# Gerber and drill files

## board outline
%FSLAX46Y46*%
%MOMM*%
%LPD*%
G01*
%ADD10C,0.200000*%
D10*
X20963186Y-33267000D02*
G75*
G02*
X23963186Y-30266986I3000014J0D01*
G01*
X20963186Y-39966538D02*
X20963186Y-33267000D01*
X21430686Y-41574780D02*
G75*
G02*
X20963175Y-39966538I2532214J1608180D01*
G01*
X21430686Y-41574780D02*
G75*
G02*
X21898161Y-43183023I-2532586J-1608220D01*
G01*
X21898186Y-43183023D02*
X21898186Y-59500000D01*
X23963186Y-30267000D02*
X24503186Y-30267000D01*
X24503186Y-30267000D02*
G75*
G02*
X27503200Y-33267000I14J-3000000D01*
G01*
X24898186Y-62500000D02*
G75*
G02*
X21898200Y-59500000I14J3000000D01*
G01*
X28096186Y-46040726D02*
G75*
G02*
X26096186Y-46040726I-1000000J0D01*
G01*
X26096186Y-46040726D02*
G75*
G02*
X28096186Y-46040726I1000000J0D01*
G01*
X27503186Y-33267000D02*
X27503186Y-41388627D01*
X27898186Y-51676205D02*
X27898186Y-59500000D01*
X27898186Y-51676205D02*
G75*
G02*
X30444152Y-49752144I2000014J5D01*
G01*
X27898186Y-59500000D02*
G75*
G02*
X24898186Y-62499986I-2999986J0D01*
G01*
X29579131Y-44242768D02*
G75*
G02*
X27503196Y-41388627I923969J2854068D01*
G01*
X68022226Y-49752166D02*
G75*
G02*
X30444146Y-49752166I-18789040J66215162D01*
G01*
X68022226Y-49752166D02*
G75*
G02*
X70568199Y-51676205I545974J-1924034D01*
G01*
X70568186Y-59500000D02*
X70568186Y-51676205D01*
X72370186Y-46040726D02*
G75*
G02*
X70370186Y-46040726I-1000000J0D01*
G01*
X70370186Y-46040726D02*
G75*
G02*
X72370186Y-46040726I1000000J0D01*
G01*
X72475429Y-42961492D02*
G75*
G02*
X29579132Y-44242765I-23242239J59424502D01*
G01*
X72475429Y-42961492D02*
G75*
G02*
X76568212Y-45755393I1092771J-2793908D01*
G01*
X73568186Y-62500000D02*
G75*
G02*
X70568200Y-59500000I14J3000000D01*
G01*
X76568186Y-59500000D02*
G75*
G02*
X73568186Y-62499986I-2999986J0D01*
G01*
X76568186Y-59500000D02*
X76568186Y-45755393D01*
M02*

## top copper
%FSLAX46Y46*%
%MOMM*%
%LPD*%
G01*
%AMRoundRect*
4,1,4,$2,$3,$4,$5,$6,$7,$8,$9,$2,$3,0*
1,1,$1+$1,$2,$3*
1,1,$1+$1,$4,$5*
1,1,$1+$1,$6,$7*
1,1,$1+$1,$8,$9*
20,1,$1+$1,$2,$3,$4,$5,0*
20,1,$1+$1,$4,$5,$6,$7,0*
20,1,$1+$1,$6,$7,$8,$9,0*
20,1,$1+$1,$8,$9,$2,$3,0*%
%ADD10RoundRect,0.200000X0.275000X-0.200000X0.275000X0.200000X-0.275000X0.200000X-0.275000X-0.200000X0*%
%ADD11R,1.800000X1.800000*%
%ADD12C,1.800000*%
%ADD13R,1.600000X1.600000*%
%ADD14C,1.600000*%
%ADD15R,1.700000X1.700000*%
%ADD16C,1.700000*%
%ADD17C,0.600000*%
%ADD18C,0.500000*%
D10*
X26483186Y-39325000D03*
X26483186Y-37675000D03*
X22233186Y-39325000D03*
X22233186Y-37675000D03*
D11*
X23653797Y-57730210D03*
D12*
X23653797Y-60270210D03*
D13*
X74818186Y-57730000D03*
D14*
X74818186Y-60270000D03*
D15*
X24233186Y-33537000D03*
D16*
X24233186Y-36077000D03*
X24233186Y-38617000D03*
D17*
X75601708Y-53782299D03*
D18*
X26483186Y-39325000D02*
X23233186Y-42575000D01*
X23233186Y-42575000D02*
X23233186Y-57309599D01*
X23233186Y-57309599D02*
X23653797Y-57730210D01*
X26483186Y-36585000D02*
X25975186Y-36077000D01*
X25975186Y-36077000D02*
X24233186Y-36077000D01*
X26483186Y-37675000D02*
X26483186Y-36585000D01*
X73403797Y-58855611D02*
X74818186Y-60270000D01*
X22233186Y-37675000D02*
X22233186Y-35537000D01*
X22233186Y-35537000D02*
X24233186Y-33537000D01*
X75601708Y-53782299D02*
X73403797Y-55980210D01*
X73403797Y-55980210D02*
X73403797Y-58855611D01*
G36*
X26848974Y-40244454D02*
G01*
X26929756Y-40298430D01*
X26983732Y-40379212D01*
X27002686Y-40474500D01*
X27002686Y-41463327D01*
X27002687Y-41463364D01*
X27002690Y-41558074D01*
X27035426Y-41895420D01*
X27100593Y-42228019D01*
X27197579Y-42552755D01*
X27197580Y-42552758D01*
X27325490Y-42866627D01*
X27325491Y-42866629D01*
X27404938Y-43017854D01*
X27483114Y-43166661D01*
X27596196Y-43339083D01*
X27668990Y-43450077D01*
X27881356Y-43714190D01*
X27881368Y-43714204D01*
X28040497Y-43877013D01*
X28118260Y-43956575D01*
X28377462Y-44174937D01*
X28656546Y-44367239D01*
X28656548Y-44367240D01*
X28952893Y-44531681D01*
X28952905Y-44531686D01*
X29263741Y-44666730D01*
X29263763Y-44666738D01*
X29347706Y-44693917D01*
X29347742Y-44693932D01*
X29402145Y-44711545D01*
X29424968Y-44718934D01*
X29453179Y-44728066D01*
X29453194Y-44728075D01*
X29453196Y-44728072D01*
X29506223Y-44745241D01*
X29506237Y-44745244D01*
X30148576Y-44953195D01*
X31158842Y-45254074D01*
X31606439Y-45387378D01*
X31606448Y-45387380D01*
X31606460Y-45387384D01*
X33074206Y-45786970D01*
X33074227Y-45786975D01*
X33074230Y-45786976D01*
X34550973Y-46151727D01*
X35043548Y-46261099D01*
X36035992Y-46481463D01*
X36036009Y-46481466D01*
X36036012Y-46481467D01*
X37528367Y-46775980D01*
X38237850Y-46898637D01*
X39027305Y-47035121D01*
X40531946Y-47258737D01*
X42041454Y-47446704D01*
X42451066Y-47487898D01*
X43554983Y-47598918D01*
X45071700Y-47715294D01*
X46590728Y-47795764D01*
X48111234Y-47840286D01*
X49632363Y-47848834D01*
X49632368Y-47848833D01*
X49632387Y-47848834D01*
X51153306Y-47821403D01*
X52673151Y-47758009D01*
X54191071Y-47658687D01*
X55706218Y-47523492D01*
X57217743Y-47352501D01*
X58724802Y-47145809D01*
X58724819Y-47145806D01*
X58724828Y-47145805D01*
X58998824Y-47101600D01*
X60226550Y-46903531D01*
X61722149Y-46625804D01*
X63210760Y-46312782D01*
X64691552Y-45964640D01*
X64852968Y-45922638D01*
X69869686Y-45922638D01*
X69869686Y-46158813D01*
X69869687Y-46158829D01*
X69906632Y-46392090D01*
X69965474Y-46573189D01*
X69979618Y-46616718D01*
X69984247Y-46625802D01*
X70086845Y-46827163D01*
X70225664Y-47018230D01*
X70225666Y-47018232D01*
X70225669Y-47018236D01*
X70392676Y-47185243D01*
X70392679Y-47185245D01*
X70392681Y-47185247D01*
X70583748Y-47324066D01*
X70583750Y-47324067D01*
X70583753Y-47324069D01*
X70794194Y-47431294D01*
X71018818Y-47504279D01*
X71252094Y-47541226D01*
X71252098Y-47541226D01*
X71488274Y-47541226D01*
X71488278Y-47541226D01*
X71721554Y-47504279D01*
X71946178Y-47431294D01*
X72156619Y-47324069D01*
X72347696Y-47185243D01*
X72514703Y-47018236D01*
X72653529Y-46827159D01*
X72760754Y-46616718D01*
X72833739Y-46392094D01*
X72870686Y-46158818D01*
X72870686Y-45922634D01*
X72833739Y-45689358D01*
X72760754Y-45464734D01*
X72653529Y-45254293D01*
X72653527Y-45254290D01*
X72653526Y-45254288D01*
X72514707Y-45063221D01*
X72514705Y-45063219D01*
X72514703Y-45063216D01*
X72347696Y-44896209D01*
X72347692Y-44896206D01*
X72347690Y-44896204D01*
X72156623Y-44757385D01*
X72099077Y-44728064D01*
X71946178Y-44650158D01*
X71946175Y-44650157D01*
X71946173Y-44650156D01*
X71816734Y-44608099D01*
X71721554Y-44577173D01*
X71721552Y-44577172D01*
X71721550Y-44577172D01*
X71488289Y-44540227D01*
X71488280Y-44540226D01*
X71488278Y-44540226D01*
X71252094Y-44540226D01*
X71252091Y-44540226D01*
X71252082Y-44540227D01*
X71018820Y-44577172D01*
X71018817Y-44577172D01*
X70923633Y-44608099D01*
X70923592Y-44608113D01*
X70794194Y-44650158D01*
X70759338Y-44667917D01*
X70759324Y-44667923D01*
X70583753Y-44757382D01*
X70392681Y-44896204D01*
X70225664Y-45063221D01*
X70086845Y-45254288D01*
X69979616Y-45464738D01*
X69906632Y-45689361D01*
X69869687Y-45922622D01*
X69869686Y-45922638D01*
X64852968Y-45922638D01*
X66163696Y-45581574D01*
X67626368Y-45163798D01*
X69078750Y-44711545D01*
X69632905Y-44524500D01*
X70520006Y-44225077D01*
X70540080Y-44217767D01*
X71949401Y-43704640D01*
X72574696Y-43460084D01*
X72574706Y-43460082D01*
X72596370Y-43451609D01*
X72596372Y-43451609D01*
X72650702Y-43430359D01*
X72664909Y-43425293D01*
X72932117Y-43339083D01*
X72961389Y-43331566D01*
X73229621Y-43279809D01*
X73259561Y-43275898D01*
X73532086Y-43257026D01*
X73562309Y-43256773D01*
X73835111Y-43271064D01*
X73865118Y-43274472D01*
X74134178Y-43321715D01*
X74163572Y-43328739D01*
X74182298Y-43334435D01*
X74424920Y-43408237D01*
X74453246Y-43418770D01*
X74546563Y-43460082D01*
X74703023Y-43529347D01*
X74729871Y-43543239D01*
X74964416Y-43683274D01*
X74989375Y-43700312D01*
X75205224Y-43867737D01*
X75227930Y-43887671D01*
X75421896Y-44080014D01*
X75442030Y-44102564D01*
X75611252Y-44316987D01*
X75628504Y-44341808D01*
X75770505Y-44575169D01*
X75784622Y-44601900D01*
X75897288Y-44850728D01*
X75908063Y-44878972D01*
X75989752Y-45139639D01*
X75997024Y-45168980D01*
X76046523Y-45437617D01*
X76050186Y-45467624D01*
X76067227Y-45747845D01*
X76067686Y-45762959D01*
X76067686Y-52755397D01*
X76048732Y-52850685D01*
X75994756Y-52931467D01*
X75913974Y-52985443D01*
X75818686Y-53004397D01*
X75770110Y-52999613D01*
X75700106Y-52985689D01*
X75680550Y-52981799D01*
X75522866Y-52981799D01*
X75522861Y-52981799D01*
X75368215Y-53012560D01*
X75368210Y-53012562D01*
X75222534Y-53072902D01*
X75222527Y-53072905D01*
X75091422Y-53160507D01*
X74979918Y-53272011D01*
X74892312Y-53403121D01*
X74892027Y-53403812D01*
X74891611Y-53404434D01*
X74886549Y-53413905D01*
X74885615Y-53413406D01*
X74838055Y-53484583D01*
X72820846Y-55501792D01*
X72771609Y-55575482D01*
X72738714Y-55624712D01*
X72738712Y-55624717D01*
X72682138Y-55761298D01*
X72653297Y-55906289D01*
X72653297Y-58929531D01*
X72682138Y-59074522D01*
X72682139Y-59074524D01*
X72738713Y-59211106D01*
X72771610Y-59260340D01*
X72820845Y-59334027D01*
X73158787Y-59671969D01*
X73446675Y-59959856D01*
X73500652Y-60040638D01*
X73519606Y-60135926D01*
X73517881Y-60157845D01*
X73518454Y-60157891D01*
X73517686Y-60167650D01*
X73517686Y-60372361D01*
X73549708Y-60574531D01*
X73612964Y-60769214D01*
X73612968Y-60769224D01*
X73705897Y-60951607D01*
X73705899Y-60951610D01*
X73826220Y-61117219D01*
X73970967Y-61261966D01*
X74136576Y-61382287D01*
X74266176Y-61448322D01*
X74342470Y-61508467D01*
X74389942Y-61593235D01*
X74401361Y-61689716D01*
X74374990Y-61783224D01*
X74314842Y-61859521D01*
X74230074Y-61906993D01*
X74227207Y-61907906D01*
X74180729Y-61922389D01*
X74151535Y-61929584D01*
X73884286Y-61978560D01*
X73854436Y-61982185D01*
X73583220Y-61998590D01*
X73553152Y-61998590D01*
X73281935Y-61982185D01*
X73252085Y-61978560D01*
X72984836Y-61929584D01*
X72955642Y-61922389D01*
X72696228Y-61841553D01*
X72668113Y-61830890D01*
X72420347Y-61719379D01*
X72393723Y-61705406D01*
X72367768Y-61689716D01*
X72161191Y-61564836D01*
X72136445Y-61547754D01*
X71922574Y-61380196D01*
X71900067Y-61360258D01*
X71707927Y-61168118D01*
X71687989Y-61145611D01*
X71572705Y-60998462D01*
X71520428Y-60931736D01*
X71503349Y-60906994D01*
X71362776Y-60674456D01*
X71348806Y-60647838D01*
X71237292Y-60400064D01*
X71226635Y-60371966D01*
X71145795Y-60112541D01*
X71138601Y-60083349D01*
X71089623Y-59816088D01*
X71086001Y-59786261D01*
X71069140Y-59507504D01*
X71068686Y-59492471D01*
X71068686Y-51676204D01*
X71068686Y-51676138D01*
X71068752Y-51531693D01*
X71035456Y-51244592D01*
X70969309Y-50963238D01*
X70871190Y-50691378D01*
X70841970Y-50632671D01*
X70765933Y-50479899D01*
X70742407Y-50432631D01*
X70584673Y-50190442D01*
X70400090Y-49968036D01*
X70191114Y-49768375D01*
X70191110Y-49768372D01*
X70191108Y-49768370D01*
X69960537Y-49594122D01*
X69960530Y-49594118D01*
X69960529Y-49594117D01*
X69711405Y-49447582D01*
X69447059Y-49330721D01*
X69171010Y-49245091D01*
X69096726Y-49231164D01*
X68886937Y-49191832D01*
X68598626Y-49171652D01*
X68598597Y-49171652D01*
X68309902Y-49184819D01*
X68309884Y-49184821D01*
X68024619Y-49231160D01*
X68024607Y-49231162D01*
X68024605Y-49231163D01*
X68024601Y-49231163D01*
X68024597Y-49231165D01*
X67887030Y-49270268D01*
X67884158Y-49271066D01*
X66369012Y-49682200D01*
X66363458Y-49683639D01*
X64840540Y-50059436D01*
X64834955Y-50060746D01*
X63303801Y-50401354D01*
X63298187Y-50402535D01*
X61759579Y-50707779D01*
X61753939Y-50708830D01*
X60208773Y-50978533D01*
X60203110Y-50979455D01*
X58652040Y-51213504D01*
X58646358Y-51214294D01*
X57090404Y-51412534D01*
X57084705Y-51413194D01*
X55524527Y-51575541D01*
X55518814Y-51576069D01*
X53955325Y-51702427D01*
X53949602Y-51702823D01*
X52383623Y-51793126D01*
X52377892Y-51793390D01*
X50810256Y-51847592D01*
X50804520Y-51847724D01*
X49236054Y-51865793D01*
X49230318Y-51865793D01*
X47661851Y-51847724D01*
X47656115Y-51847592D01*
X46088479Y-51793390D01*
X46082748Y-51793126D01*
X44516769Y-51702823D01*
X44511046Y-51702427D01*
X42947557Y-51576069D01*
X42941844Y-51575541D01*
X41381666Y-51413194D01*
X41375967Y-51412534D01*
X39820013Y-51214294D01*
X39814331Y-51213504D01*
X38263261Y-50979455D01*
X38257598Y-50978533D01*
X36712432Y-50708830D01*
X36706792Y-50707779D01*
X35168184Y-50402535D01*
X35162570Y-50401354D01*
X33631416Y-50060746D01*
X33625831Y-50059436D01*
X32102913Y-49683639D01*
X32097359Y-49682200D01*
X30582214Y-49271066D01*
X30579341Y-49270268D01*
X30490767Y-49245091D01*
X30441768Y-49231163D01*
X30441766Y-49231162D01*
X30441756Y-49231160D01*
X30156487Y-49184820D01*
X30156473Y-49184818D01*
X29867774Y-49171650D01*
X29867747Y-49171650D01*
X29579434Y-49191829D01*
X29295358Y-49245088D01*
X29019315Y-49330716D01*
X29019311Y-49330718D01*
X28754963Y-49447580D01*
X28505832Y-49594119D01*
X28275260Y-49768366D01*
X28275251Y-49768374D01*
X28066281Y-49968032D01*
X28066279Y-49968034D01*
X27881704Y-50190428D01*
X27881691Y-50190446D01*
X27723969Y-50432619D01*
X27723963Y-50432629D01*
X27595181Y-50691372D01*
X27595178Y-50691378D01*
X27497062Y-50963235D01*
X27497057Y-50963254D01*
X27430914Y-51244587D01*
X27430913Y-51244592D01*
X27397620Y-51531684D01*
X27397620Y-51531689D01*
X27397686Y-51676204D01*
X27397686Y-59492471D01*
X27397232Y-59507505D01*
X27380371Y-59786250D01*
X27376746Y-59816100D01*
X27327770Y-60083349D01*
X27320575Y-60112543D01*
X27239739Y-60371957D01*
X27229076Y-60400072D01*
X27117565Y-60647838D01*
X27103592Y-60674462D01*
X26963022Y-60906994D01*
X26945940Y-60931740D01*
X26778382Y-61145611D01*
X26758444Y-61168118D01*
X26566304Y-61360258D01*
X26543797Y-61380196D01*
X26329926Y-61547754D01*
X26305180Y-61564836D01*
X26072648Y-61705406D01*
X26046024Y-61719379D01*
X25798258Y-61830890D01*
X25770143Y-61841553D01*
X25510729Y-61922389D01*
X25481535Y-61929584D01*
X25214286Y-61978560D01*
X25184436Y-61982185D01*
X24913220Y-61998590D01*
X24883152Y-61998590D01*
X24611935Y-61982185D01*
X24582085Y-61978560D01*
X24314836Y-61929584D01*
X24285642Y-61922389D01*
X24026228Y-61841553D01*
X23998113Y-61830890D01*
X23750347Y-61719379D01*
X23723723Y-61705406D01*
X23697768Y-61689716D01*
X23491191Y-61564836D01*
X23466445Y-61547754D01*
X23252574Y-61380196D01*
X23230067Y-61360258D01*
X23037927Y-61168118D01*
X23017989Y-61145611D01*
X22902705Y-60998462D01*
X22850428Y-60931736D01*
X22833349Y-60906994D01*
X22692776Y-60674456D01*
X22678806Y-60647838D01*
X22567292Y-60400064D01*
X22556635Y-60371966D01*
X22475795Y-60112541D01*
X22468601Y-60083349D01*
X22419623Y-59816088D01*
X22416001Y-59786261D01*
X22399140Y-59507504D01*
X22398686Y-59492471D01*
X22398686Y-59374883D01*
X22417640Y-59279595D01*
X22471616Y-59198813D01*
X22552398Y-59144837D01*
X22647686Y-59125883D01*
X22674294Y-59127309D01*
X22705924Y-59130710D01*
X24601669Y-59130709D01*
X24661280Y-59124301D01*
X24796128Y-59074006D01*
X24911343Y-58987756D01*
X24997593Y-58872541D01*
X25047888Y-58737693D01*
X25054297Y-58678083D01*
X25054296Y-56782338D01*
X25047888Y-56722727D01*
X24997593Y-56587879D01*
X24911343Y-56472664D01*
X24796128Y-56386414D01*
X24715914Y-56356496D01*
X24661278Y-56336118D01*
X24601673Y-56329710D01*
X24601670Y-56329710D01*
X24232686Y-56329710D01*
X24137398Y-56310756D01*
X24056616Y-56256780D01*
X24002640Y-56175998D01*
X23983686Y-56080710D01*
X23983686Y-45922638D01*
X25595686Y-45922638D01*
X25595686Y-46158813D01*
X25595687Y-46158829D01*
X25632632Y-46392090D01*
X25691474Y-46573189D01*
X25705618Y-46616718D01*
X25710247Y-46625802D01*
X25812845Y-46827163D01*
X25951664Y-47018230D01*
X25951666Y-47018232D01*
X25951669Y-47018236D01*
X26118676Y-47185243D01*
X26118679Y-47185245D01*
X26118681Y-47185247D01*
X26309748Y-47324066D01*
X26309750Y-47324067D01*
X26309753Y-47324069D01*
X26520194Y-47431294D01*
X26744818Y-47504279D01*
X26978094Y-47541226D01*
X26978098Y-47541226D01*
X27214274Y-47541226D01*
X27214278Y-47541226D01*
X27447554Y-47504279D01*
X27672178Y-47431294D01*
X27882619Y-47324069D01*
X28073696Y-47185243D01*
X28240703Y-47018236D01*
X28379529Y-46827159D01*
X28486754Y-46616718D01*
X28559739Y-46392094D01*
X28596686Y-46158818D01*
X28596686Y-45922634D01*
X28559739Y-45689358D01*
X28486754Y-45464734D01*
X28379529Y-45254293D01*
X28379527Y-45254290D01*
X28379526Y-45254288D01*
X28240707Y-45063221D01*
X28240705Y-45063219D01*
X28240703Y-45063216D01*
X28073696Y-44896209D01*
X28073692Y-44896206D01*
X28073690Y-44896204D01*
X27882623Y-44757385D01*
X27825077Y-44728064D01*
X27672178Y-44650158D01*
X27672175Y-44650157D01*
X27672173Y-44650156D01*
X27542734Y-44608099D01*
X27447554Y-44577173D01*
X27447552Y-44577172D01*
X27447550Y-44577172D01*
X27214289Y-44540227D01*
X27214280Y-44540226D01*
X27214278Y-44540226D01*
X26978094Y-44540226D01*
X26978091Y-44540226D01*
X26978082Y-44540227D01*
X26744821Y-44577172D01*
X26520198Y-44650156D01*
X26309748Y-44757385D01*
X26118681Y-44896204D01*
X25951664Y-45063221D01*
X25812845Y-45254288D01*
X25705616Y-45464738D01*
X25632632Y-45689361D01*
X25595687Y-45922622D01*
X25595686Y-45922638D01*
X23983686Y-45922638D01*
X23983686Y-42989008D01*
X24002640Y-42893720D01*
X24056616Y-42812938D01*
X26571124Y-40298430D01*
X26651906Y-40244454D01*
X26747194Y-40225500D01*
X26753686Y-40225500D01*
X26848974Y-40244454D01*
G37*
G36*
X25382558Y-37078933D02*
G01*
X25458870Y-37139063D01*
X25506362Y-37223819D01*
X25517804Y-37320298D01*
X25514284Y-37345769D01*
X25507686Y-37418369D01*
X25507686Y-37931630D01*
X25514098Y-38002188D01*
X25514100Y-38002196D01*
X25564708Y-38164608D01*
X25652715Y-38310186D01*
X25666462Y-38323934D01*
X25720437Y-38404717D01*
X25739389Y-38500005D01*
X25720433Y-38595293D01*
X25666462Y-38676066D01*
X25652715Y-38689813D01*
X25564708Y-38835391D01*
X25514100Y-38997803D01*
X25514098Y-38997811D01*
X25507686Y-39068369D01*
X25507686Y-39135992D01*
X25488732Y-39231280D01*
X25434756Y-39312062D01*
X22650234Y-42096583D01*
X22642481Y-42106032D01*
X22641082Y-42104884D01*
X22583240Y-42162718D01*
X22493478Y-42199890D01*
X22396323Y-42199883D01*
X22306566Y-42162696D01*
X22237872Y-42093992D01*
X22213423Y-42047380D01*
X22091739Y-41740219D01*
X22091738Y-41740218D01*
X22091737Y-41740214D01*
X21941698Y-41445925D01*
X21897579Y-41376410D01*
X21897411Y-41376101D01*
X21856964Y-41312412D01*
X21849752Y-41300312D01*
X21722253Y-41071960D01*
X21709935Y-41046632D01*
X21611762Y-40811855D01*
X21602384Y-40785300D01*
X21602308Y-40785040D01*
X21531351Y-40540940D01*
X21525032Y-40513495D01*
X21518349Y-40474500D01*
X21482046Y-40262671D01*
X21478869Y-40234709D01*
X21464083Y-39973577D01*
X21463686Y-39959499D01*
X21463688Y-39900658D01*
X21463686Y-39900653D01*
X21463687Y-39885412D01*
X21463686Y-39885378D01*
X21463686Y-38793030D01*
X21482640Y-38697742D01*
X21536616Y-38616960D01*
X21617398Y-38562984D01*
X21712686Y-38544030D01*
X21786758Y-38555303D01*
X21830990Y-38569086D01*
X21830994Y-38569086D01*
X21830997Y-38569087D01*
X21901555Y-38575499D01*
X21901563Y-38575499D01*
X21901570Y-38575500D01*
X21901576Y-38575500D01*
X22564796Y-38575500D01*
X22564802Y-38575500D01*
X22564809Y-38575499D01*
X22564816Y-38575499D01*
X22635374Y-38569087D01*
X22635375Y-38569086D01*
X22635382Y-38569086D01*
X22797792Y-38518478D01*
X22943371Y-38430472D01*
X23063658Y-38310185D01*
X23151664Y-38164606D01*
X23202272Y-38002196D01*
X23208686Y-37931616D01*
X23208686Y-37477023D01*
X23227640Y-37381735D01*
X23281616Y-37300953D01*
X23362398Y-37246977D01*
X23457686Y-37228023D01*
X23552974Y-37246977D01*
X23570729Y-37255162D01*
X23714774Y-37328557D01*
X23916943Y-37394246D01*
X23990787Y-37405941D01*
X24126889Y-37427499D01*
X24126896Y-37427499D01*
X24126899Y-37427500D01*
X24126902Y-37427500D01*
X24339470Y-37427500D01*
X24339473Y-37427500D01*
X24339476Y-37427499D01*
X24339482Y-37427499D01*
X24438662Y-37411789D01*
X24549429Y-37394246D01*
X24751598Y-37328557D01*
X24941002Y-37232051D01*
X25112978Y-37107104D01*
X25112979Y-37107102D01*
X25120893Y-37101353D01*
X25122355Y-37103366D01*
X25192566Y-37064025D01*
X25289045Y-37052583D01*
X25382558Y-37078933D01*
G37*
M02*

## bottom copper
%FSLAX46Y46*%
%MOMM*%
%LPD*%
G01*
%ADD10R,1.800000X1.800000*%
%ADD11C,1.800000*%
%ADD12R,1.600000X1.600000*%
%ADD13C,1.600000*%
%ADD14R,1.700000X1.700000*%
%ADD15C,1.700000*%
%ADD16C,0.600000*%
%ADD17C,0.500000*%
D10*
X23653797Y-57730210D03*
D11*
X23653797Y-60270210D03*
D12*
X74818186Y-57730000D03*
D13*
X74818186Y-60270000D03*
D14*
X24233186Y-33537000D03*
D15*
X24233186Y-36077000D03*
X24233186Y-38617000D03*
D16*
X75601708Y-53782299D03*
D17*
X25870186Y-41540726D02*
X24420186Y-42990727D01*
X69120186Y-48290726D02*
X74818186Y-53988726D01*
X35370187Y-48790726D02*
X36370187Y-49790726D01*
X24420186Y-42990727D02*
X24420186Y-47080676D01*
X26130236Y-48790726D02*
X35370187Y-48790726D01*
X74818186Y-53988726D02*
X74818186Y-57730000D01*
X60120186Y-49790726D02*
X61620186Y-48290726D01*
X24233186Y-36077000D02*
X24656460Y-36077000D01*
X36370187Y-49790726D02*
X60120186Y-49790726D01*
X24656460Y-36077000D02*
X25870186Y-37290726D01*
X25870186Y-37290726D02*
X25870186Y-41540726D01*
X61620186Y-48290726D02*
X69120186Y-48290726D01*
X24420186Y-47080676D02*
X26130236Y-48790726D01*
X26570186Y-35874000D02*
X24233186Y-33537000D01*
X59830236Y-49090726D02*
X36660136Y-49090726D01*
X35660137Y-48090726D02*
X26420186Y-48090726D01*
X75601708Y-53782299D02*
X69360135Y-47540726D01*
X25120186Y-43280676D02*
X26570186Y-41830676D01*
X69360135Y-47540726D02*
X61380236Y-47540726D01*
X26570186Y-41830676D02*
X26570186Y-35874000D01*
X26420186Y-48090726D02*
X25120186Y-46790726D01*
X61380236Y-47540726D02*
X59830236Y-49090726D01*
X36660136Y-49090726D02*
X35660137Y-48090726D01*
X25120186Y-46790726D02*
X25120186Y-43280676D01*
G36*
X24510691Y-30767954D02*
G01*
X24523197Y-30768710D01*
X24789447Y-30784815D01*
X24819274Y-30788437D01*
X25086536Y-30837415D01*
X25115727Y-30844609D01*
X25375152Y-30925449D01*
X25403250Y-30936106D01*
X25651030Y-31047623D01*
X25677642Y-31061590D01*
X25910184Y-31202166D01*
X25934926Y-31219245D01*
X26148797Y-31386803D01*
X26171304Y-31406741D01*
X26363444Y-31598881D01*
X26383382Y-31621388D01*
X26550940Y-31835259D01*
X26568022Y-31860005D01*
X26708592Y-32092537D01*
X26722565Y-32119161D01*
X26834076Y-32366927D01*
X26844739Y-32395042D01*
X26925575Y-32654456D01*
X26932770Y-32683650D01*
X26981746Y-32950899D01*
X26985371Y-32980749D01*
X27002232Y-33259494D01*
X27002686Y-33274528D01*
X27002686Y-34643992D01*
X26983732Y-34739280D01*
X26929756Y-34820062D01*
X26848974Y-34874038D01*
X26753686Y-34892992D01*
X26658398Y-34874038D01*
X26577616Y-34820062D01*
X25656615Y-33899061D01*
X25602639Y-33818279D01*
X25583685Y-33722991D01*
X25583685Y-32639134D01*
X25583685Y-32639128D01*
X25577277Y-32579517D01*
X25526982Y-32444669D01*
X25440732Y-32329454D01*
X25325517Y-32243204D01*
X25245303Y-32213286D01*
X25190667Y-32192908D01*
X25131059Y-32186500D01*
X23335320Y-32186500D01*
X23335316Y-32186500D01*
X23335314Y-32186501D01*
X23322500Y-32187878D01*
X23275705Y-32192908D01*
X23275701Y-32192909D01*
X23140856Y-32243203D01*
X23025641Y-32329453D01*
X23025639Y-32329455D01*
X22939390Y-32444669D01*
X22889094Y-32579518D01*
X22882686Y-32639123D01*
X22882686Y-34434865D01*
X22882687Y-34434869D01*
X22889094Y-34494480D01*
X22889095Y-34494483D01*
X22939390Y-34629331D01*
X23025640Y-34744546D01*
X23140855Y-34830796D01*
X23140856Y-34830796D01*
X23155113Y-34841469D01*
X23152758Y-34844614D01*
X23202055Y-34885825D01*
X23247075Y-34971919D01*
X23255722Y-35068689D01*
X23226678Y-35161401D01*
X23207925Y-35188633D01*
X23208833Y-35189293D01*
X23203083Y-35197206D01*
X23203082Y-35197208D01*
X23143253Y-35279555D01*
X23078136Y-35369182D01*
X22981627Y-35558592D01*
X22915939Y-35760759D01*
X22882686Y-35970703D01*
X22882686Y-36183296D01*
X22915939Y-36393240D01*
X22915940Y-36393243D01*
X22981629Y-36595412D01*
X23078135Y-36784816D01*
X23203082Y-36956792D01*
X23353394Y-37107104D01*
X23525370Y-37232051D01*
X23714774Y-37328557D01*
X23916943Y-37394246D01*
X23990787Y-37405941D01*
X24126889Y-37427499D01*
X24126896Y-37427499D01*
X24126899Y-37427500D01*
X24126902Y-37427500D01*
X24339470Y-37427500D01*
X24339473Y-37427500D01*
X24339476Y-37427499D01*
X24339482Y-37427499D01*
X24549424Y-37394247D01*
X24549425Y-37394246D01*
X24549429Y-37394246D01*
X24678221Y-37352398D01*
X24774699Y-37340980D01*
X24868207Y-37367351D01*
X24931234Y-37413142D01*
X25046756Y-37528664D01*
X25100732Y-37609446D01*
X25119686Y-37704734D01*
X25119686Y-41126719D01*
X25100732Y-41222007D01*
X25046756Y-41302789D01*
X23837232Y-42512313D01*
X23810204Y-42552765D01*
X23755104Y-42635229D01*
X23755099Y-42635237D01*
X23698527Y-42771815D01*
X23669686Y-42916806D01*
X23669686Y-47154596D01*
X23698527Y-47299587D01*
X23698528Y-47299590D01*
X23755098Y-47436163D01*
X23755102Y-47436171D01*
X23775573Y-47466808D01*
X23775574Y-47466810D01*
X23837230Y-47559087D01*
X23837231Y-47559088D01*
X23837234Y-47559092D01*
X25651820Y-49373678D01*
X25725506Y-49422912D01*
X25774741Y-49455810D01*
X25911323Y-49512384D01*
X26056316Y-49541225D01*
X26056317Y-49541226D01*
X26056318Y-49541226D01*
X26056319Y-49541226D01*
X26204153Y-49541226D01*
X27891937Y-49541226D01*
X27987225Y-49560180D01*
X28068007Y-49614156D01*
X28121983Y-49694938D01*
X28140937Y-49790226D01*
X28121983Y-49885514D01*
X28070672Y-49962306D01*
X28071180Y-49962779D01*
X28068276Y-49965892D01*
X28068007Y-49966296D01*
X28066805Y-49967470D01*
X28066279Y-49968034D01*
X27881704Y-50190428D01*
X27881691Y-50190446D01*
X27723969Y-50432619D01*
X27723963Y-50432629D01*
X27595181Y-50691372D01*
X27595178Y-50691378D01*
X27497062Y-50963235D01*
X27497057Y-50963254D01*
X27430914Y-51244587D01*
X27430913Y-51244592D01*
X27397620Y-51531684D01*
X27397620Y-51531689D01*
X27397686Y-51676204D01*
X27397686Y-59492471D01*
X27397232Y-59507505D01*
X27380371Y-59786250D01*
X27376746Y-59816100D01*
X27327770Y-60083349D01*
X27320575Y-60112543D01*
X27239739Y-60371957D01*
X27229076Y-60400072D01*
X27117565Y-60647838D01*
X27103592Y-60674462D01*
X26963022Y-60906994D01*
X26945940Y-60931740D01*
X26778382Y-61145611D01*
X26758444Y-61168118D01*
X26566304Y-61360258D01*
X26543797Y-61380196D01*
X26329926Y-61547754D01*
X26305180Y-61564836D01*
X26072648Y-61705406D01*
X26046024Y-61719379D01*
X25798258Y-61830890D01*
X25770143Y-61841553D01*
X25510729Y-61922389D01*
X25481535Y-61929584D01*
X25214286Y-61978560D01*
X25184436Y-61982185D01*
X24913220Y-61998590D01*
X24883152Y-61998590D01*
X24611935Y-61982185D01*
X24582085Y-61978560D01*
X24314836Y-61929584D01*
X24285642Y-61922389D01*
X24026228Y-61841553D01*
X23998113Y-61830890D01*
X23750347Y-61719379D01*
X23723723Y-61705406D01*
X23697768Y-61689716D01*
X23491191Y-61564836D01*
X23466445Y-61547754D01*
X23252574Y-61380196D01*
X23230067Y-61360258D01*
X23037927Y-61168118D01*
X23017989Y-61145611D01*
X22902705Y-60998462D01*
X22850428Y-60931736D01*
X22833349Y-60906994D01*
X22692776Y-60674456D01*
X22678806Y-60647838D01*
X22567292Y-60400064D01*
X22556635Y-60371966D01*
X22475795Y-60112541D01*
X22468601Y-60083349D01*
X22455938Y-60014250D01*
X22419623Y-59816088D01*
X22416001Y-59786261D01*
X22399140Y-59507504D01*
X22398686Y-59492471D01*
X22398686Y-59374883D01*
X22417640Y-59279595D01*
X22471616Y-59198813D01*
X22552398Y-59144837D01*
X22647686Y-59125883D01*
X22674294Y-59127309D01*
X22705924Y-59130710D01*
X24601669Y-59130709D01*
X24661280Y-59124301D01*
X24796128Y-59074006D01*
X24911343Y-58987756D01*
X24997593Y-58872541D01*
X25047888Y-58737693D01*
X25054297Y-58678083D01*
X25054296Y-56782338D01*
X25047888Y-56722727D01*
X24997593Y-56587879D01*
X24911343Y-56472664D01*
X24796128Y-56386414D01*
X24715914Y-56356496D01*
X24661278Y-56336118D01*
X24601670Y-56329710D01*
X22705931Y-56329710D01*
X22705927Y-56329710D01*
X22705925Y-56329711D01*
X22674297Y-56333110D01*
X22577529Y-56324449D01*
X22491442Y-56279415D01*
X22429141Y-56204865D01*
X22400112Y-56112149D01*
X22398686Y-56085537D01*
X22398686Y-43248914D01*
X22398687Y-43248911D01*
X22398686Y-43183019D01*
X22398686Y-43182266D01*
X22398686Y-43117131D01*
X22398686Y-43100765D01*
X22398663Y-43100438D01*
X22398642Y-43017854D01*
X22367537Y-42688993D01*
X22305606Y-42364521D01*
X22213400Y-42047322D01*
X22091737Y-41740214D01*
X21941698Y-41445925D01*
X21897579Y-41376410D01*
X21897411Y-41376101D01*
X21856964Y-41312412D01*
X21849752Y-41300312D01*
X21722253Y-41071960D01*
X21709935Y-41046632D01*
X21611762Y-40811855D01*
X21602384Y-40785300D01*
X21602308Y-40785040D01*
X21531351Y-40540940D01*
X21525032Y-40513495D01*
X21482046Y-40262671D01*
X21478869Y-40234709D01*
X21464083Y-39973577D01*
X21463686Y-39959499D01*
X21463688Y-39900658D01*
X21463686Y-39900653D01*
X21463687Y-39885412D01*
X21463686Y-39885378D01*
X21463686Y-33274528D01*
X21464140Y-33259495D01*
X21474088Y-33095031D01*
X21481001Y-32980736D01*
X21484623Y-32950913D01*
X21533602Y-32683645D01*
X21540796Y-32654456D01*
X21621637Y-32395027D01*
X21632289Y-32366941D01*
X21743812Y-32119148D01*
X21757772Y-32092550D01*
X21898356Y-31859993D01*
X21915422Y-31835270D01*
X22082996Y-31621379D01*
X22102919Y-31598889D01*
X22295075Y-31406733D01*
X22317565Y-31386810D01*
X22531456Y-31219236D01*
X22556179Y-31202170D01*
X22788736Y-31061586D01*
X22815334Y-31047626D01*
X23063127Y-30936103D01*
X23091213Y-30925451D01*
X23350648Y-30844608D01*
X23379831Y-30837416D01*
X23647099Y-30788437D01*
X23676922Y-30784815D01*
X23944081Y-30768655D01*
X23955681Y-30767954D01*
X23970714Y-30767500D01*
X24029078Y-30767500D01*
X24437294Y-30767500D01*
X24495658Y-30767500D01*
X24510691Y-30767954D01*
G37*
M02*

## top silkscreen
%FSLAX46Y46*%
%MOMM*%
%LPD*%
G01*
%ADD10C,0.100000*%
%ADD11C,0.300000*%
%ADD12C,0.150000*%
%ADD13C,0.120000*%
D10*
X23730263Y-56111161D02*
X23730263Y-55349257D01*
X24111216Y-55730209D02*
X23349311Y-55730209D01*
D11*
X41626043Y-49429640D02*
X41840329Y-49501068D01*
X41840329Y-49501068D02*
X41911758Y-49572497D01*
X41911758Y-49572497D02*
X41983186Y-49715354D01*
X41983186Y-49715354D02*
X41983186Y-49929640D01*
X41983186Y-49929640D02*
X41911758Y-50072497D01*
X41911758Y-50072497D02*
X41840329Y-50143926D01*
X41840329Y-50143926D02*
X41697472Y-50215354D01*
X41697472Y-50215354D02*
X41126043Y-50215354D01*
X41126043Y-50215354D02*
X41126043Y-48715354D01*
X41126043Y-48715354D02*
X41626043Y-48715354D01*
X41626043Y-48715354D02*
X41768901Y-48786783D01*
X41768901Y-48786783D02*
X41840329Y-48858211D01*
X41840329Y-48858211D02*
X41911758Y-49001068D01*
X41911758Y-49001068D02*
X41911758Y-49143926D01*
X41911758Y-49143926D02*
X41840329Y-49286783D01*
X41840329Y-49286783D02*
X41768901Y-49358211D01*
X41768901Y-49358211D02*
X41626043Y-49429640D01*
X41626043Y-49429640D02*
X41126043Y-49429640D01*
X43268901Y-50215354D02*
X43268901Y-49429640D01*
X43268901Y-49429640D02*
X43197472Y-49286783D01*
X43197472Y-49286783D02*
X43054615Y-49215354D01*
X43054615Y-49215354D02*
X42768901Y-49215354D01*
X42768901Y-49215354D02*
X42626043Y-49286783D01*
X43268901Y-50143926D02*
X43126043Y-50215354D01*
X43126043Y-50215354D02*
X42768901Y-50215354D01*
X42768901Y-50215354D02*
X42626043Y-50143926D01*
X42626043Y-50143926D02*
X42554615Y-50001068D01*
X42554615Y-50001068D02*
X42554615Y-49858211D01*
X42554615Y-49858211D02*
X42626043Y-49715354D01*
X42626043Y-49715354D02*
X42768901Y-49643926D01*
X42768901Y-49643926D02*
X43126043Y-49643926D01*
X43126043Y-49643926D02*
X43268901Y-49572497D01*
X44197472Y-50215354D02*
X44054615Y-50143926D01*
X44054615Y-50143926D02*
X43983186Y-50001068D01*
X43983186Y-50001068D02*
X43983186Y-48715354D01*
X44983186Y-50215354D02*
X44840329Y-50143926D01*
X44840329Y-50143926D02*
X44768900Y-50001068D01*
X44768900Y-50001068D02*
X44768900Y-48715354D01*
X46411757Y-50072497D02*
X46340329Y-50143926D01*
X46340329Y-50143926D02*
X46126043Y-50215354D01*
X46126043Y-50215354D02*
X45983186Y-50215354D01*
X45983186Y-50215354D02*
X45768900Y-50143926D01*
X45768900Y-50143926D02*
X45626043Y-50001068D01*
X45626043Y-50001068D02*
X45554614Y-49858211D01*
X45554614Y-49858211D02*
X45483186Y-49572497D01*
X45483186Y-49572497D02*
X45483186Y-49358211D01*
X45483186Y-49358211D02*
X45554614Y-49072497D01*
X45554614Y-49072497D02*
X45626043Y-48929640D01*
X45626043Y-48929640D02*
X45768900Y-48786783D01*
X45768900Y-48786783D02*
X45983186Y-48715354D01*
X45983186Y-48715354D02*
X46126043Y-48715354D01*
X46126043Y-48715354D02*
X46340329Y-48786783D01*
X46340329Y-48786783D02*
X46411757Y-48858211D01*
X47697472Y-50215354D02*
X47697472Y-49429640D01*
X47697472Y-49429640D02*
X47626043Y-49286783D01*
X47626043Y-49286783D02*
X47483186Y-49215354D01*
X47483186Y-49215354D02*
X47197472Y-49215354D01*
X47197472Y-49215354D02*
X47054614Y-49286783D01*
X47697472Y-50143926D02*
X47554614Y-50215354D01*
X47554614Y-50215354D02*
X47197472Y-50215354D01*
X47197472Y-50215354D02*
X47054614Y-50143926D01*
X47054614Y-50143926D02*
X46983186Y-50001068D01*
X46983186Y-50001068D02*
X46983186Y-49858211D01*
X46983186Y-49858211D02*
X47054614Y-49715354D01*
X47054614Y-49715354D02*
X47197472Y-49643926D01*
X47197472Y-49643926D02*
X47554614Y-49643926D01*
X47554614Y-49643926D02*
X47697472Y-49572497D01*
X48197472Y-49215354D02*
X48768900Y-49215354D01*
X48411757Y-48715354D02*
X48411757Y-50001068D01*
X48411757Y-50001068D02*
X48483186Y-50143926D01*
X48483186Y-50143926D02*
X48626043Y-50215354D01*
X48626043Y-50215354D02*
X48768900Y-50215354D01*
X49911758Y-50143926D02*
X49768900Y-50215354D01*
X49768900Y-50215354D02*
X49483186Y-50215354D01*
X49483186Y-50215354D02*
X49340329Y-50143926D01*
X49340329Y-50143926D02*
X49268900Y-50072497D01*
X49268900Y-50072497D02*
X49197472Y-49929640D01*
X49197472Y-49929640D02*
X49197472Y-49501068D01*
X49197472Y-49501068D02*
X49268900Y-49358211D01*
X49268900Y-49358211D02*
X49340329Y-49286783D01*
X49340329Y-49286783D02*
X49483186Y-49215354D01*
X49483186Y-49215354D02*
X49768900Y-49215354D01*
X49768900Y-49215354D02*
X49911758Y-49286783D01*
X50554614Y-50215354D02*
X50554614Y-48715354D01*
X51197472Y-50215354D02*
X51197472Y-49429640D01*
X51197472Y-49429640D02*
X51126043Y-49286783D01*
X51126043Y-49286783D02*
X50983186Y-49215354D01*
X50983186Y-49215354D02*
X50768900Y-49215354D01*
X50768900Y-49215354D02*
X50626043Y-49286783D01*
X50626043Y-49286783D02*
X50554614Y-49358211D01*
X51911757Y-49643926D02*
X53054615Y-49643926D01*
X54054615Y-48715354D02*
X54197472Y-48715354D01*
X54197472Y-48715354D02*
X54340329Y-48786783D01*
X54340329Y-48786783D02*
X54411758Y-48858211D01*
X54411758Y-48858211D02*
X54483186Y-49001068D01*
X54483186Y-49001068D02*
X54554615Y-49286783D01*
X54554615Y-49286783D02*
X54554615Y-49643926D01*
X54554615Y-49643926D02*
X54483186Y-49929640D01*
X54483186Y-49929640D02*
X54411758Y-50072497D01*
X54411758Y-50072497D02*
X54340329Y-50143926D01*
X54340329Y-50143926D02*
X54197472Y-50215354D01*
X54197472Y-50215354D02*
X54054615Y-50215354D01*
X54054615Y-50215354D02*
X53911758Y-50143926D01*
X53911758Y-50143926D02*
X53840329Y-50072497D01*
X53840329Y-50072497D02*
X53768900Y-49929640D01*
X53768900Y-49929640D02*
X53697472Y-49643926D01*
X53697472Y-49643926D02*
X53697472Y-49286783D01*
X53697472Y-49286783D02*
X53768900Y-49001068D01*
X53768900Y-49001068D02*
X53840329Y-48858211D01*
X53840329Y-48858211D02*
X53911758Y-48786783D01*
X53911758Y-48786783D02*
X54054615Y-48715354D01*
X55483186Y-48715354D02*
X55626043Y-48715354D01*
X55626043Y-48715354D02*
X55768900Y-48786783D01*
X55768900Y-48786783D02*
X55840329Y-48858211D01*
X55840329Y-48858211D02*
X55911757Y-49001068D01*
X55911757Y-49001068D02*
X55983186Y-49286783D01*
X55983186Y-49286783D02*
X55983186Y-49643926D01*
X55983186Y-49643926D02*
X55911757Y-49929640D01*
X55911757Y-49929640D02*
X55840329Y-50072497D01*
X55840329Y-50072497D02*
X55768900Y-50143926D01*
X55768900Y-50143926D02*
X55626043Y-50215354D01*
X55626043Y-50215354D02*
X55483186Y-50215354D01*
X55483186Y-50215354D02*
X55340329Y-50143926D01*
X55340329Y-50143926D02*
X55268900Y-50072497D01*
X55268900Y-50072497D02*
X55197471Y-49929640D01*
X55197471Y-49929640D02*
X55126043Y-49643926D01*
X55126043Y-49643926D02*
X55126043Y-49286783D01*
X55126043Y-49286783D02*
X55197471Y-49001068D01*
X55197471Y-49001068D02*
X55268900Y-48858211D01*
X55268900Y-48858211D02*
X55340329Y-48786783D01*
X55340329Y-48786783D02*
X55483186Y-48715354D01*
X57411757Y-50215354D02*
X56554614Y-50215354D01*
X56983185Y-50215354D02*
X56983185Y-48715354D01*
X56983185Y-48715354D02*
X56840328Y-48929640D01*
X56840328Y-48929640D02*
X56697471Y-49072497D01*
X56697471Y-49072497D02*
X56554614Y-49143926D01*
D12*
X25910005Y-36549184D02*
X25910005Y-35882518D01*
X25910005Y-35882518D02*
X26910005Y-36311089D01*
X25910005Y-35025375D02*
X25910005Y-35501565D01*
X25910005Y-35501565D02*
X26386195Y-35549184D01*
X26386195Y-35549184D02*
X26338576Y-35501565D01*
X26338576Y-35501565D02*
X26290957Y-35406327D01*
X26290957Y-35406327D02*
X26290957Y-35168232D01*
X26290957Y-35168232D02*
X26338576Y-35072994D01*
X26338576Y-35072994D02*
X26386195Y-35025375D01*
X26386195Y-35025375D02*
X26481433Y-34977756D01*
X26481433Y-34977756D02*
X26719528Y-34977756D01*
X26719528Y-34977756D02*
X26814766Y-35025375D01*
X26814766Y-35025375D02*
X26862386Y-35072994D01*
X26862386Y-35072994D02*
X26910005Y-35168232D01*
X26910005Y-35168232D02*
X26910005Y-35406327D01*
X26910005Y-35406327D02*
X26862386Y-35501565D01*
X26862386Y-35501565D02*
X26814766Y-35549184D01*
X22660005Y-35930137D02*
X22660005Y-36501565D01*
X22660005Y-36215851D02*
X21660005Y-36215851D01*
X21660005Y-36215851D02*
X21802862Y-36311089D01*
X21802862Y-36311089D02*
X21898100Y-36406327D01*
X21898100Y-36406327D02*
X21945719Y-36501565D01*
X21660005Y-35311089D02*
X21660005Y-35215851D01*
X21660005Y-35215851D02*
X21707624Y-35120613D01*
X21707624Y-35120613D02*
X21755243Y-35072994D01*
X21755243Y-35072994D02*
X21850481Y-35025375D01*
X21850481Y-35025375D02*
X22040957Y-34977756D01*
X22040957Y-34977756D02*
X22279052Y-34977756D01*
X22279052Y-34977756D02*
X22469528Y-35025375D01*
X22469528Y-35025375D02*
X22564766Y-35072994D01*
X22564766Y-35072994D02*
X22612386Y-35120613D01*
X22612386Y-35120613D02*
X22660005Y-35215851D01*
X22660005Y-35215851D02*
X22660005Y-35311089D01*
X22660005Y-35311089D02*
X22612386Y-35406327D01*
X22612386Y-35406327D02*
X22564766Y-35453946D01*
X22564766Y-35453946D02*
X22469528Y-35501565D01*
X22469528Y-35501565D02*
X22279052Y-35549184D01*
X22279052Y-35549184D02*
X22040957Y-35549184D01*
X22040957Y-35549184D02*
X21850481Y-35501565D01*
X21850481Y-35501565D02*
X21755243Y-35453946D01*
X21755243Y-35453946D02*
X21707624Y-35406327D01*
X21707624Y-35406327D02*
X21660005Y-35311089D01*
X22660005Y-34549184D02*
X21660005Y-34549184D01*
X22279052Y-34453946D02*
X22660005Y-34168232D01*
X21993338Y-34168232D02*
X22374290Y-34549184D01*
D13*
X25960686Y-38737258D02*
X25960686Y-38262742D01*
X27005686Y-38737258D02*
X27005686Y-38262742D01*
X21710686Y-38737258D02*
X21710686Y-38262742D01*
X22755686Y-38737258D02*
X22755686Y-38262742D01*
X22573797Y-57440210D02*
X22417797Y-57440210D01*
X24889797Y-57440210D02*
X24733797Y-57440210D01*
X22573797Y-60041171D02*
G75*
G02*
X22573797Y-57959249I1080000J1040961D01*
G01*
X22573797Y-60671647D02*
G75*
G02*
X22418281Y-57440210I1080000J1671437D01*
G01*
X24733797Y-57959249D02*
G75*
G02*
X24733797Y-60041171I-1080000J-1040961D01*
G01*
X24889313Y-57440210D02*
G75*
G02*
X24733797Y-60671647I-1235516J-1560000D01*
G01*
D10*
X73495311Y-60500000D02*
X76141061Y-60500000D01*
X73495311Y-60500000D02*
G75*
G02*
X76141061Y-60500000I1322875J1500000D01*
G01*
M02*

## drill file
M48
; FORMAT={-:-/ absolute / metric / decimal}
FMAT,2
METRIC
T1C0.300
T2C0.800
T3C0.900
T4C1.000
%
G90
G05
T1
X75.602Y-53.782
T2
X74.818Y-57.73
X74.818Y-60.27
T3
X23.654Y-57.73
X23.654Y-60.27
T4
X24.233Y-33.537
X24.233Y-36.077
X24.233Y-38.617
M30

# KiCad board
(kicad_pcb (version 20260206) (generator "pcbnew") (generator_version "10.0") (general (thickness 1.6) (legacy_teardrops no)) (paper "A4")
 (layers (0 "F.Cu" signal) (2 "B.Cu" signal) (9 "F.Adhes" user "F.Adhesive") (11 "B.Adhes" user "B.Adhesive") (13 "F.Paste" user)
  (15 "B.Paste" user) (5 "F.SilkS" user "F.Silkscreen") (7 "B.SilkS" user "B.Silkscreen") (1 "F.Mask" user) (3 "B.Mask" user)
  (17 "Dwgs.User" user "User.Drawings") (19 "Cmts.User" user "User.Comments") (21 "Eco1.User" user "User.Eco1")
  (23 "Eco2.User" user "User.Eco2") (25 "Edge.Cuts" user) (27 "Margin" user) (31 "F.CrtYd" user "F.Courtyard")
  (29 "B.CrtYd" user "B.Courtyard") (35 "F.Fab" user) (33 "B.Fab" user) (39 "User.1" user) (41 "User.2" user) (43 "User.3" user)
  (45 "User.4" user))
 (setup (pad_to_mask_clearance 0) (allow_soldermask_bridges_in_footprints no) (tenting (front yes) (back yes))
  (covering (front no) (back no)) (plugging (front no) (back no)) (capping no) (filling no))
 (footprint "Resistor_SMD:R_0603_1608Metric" (layer "F.Cu") (at 26.483186 38.5 90)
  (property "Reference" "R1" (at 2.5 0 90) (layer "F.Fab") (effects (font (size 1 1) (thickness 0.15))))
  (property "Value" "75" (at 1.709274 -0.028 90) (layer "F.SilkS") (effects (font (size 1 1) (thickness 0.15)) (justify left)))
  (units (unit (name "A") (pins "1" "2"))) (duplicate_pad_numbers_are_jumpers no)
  (fp_line (start -0.237258 -0.5225) (end 0.237258 -0.5225) (stroke (width 0.12) (type solid)) (layer "F.SilkS"))
  (fp_line (start -0.237258 0.5225) (end 0.237258 0.5225) (stroke (width 0.12) (type solid)) (layer "F.SilkS"))
  (pad "1" smd roundrect (at -0.825 0 90) (size 0.8 0.95) (layers "F.Cu" "F.Mask" "F.Paste") (roundrect_rratio 0.25) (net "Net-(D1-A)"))
  (pad "2" smd roundrect (at 0.825 0 90) (size 0.8 0.95) (layers "F.Cu" "F.Mask" "F.Paste") (roundrect_rratio 0.25) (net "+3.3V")))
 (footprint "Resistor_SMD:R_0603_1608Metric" (layer "F.Cu") (at 22.233186 38.5 90)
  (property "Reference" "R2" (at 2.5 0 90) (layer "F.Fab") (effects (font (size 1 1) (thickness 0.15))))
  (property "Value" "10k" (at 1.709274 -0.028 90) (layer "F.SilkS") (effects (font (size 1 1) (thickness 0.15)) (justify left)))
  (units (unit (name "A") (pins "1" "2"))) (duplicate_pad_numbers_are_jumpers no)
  (fp_line (start -0.237258 -0.5225) (end 0.237258 -0.5225) (stroke (width 0.12) (type solid)) (layer "F.SilkS"))
  (fp_line (start -0.237258 0.5225) (end 0.237258 0.5225) (stroke (width 0.12) (type solid)) (layer "F.SilkS"))
  (pad "1" smd roundrect (at -0.825 0 90) (size 0.8 0.95) (layers "F.Cu" "F.Mask" "F.Paste") (roundrect_rratio 0.25) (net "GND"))
  (pad "2" smd roundrect (at 0.825 0 90) (size 0.8 0.95) (layers "F.Cu" "F.Mask" "F.Paste") (roundrect_rratio 0.25) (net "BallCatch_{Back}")))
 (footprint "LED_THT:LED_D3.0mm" (layer "F.Cu") (at 23.653797 57.73021 -90)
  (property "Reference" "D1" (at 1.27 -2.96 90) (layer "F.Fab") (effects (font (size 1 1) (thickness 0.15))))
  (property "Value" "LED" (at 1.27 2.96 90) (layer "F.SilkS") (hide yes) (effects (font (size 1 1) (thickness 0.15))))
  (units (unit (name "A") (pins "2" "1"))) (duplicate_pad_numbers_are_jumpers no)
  (fp_line (start -0.29 1.08) (end -0.29 1.236) (stroke (width 0.12) (type solid)) (layer "F.SilkS"))
  (fp_line (start -0.29 -1.236) (end -0.29 -1.08) (stroke (width 0.12) (type solid)) (layer "F.SilkS"))
  (fp_arc (start 2.310961 1.08) (mid 1.27 1.5) (end 0.229039 1.08) (stroke (width 0.12) (type solid)) (layer "F.SilkS"))
  (fp_arc (start 2.941437 1.08) (mid 1.36566 1.987699) (end -0.29 1.235516) (stroke (width 0.12) (type solid)) (layer "F.SilkS"))
  (fp_arc (start 0.229039 -1.08) (mid 1.27 -1.5) (end 2.310961 -1.08) (stroke (width 0.12) (type solid)) (layer "F.SilkS"))
  (fp_arc (start -0.29 -1.235516) (mid 1.36566 -1.987699) (end 2.941437 -1.08) (stroke (width 0.12) (type solid)) (layer "F.SilkS"))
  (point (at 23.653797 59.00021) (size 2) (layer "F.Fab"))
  (pad "1" thru_hole rect (at 0 0 270) (size 1.8 1.8) (drill 0.9) (layers "*.Cu" "*.Mask") (remove_unused_layers no) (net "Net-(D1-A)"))
  (pad "2" thru_hole circle (at 2.54 0 270) (size 1.8 1.8) (drill 0.9) (layers "*.Cu" "*.Mask") (remove_unused_layers no) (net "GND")))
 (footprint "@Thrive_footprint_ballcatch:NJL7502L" (layer "F.Cu") (at 74.818186 59 90)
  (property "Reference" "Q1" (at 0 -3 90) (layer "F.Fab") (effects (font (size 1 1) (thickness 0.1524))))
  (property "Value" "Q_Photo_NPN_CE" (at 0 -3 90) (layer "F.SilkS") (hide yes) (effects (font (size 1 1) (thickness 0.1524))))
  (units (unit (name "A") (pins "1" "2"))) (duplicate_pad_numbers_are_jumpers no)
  (fp_line (start -1.5 -1.322875) (end -1.5 1.322875) (stroke (width 0.1) (type default)) (layer "F.SilkS"))
  (fp_arc (start -1.5 -1.322875) (mid 2 0) (end -1.5 1.322875) (stroke (width 0.1) (type default)) (layer "F.SilkS"))
  (pad "1" thru_hole rect (at 1.27 0 180) (size 1.6 1.6) (drill 0.8) (layers "*.Cu" "*.Mask") (remove_unused_layers no) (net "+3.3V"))
  (pad "2" thru_hole circle (at -1.27 0 180) (size 1.6 1.6) (drill 0.8) (layers "*.Cu" "*.Mask") (remove_unused_layers no)
   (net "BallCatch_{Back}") (thermal_bridge_angle 90)))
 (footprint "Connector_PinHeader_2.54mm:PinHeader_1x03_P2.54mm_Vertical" (layer "B.Cu") (at 24.233186 33.537 180)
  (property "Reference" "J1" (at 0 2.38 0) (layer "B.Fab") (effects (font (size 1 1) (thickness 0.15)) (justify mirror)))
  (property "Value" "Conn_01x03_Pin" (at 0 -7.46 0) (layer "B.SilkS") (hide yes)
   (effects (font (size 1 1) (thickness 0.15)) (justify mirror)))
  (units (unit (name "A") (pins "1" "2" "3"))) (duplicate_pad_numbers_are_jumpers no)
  (pad "1" thru_hole rect (at 0 0 180) (size 1.7 1.7) (drill 1) (layers "*.Cu" "*.Mask") (remove_unused_layers no) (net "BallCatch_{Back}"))
  (pad "2" thru_hole circle (at 0 -2.54 180) (size 1.7 1.7) (drill 1) (layers "*.Cu" "*.Mask") (remove_unused_layers no) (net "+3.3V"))
  (pad "3" thru_hole circle (at 0 -5.08 180) (size 1.7 1.7) (drill 1) (layers "*.Cu" "*.Mask") (remove_unused_layers no) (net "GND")))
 (gr_arc (start 20.963186 33.267) (mid 21.841866 31.14568) (end 23.963186 30.267) (stroke (width 0.2) (type default)) (layer "Edge.Cuts"))
 (gr_line (start 20.963186 39.966538) (end 20.963186 33.267) (stroke (width 0.2) (type default)) (layer "Edge.Cuts"))
 (gr_arc (start 21.430686 41.57478) (mid 21.082421 40.803946) (end 20.963186 39.966538) (stroke (width 0.2) (type default))
  (layer "Edge.Cuts"))
 (gr_arc (start 21.430686 41.57478) (mid 21.778938 42.345618) (end 21.898186 43.183023) (stroke (width 0.2) (type default))
  (layer "Edge.Cuts"))
 (gr_line (start 21.898186 43.183023) (end 21.898186 59.5) (stroke (width 0.2) (type default)) (layer "Edge.Cuts"))
 (gr_line (start 23.963186 30.267) (end 24.503186 30.267) (stroke (width 0.2) (type default)) (layer "Edge.Cuts"))
 (gr_arc (start 24.503186 30.267) (mid 26.624506 31.14568) (end 27.503186 33.267) (stroke (width 0.2) (type default)) (layer "Edge.Cuts"))
 (gr_arc (start 24.898186 62.5) (mid 22.776866 61.62132) (end 21.898186 59.5) (stroke (width 0.2) (type default)) (layer "Edge.Cuts"))
 (gr_circle (center 27.096186 46.040726) (end 26.096186 46.040726) (stroke (width 0.2) (type default)) (fill no) (layer "Edge.Cuts"))
 (gr_line (start 27.503186 33.267) (end 27.503186 41.388627) (stroke (width 0.2) (type default)) (layer "Edge.Cuts"))
 (gr_line (start 27.898186 51.676205) (end 27.898186 59.5) (stroke (width 0.2) (type default)) (layer "Edge.Cuts"))
 (gr_arc (start 27.898186 51.676205) (mid 28.692349 50.080595) (end 30.444146 49.752166) (stroke (width 0.2) (type default))
  (layer "Edge.Cuts"))
 (gr_arc (start 27.898186 59.5) (mid 27.019506 61.62132) (end 24.898186 62.5) (stroke (width 0.2) (type default)) (layer "Edge.Cuts"))
 (gr_arc (start 29.579131 44.242768) (mid 28.077051 43.153259) (end 27.503186 41.388627) (stroke (width 0.2) (type default))
  (layer "Edge.Cuts"))
 (gr_arc (start 68.022226 49.752166) (mid 49.233186 52.366327) (end 30.444146 49.752166) (stroke (width 0.2) (type default))
  (layer "Edge.Cuts"))
 (gr_arc (start 68.022226 49.752166) (mid 69.774022 50.080599) (end 70.568186 51.676205) (stroke (width 0.2) (type default))
  (layer "Edge.Cuts"))
 (gr_line (start 70.568186 59.5) (end 70.568186 51.676205) (stroke (width 0.2) (type default)) (layer "Edge.Cuts"))
 (gr_circle (center 71.370186 46.040726) (end 70.370186 46.040726) (stroke (width 0.2) (type default)) (fill no) (layer "Edge.Cuts"))
 (gr_arc (start 72.475429 42.961492) (mid 51.138229 47.316643) (end 29.579131 44.242768) (stroke (width 0.2) (type default))
  (layer "Edge.Cuts"))
 (gr_arc (start 72.475429 42.961492) (mid 75.259595 43.277665) (end 76.568186 45.755393) (stroke (width 0.2) (type default))
  (layer "Edge.Cuts"))
 (gr_arc (start 73.568186 62.5) (mid 71.446866 61.62132) (end 70.568186 59.5) (stroke (width 0.2) (type default)) (layer "Edge.Cuts"))
 (gr_arc (start 76.568186 59.5) (mid 75.689506 61.62132) (end 73.568186 62.5) (stroke (width 0.2) (type default)) (layer "Edge.Cuts"))
 (gr_line (start 76.568186 59.5) (end 76.568186 45.755393) (stroke (width 0.2) (type default)) (layer "Edge.Cuts"))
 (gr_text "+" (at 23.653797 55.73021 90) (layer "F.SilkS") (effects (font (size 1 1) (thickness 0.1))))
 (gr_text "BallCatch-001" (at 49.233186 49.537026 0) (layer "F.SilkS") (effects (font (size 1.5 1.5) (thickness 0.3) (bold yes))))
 (segment (start 26.483186 39.325) (end 23.233186 42.575) (width 0.5) (layer "F.Cu") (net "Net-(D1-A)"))
 (segment (start 23.233186 42.575) (end 23.233186 57.309599) (width 0.5) (layer "F.Cu") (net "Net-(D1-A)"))
 (segment (start 23.233186 57.309599) (end 23.653797 57.73021) (width 0.5) (layer "F.Cu") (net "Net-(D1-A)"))
 (segment (start 26.483186 36.585) (end 25.975186 36.077) (width 0.5) (layer "F.Cu") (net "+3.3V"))
 (segment (start 25.975186 36.077) (end 24.233186 36.077) (width 0.5) (layer "F.Cu") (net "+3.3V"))
 (segment (start 26.483186 37.675) (end 26.483186 36.585) (width 0.5) (layer "F.Cu") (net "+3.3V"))
 (segment (start 25.870186 41.540726) (end 24.420186 42.990727) (width 0.5) (layer "B.Cu") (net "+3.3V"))
 (segment (start 69.120186 48.290726) (end 74.818186 53.988726) (width 0.5) (layer "B.Cu") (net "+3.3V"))
 (segment (start 35.370187 48.790726) (end 36.370187 49.790726) (width 0.5) (layer "B.Cu") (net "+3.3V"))
 (segment (start 24.420186 42.990727) (end 24.420186 47.080676) (width 0.5) (layer "B.Cu") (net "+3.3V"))
 (segment (start 26.130236 48.790726) (end 35.370187 48.790726) (width 0.5) (layer "B.Cu") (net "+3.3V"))
 (segment (start 74.818186 53.988726) (end 74.818186 57.73) (width 0.5) (layer "B.Cu") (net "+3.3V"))
 (segment (start 60.120186 49.790726) (end 61.620186 48.290726) (width 0.5) (layer "B.Cu") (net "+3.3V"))
 (segment (start 24.233186 36.077) (end 24.65646 36.077) (width 0.5) (layer "B.Cu") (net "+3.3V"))
 (segment (start 36.370187 49.790726) (end 60.120186 49.790726) (width 0.5) (layer "B.Cu") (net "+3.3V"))
 (segment (start 24.65646 36.077) (end 25.870186 37.290726) (width 0.5) (layer "B.Cu") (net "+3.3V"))
 (segment (start 25.870186 37.290726) (end 25.870186 41.540726) (width 0.5) (layer "B.Cu") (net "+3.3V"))
 (segment (start 61.620186 48.290726) (end 69.120186 48.290726) (width 0.5) (layer "B.Cu") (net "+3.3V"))
 (segment (start 24.420186 47.080676) (end 26.130236 48.790726) (width 0.5) (layer "B.Cu") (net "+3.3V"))
 (segment (start 73.403797 58.855611) (end 74.818186 60.27) (width 0.5) (layer "F.Cu") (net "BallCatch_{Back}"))
 (segment (start 22.233186 37.675) (end 22.233186 35.537) (width 0.5) (layer "F.Cu") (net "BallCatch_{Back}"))
 (segment (start 22.233186 35.537) (end 24.233186 33.537) (width 0.5) (layer "F.Cu") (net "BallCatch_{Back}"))
 (segment (start 75.601708 53.782299) (end 73.403797 55.98021) (width 0.5) (layer "F.Cu") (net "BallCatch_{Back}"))
 (segment (start 73.403797 55.98021) (end 73.403797 58.855611) (width 0.5) (layer "F.Cu") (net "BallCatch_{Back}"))
 (via (at 75.601708 53.782299) (size 0.6) (drill 0.3) (layers "F.Cu" "B.Cu") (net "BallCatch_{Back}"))
 (segment (start 26.570186 35.874) (end 24.233186 33.537) (width 0.5) (layer "B.Cu") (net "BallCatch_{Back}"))
 (segment (start 59.830236 49.090726) (end 36.660136 49.090726) (width 0.5) (layer "B.Cu") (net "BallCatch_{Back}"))
 (segment (start 35.660137 48.090726) (end 26.420186 48.090726) (width 0.5) (layer "B.Cu") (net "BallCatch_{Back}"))
 (segment (start 75.601708 53.782299) (end 69.360135 47.540726) (width 0.5) (layer "B.Cu") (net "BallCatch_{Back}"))
 (segment (start 25.120186 43.280676) (end 26.570186 41.830676) (width 0.5) (layer "B.Cu") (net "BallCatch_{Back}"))
 (segment (start 69.360135 47.540726) (end 61.380236 47.540726) (width 0.5) (layer "B.Cu") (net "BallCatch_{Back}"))
 (segment (start 26.570186 41.830676) (end 26.570186 35.874) (width 0.5) (layer "B.Cu") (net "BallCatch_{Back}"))
 (segment (start 26.420186 48.090726) (end 25.120186 46.790726) (width 0.5) (layer "B.Cu") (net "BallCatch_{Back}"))
 (segment (start 61.380236 47.540726) (end 59.830236 49.090726) (width 0.5) (layer "B.Cu") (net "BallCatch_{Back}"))
 (segment (start 36.660136 49.090726) (end 35.660137 48.090726) (width 0.5) (layer "B.Cu") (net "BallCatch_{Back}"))
 (segment (start 25.120186 46.790726) (end 25.120186 43.280676) (width 0.5) (layer "B.Cu") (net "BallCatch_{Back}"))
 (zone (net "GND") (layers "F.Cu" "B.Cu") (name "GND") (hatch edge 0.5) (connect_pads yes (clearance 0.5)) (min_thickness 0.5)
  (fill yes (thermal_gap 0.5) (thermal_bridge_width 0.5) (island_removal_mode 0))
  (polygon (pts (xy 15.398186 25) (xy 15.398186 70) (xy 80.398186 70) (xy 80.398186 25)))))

